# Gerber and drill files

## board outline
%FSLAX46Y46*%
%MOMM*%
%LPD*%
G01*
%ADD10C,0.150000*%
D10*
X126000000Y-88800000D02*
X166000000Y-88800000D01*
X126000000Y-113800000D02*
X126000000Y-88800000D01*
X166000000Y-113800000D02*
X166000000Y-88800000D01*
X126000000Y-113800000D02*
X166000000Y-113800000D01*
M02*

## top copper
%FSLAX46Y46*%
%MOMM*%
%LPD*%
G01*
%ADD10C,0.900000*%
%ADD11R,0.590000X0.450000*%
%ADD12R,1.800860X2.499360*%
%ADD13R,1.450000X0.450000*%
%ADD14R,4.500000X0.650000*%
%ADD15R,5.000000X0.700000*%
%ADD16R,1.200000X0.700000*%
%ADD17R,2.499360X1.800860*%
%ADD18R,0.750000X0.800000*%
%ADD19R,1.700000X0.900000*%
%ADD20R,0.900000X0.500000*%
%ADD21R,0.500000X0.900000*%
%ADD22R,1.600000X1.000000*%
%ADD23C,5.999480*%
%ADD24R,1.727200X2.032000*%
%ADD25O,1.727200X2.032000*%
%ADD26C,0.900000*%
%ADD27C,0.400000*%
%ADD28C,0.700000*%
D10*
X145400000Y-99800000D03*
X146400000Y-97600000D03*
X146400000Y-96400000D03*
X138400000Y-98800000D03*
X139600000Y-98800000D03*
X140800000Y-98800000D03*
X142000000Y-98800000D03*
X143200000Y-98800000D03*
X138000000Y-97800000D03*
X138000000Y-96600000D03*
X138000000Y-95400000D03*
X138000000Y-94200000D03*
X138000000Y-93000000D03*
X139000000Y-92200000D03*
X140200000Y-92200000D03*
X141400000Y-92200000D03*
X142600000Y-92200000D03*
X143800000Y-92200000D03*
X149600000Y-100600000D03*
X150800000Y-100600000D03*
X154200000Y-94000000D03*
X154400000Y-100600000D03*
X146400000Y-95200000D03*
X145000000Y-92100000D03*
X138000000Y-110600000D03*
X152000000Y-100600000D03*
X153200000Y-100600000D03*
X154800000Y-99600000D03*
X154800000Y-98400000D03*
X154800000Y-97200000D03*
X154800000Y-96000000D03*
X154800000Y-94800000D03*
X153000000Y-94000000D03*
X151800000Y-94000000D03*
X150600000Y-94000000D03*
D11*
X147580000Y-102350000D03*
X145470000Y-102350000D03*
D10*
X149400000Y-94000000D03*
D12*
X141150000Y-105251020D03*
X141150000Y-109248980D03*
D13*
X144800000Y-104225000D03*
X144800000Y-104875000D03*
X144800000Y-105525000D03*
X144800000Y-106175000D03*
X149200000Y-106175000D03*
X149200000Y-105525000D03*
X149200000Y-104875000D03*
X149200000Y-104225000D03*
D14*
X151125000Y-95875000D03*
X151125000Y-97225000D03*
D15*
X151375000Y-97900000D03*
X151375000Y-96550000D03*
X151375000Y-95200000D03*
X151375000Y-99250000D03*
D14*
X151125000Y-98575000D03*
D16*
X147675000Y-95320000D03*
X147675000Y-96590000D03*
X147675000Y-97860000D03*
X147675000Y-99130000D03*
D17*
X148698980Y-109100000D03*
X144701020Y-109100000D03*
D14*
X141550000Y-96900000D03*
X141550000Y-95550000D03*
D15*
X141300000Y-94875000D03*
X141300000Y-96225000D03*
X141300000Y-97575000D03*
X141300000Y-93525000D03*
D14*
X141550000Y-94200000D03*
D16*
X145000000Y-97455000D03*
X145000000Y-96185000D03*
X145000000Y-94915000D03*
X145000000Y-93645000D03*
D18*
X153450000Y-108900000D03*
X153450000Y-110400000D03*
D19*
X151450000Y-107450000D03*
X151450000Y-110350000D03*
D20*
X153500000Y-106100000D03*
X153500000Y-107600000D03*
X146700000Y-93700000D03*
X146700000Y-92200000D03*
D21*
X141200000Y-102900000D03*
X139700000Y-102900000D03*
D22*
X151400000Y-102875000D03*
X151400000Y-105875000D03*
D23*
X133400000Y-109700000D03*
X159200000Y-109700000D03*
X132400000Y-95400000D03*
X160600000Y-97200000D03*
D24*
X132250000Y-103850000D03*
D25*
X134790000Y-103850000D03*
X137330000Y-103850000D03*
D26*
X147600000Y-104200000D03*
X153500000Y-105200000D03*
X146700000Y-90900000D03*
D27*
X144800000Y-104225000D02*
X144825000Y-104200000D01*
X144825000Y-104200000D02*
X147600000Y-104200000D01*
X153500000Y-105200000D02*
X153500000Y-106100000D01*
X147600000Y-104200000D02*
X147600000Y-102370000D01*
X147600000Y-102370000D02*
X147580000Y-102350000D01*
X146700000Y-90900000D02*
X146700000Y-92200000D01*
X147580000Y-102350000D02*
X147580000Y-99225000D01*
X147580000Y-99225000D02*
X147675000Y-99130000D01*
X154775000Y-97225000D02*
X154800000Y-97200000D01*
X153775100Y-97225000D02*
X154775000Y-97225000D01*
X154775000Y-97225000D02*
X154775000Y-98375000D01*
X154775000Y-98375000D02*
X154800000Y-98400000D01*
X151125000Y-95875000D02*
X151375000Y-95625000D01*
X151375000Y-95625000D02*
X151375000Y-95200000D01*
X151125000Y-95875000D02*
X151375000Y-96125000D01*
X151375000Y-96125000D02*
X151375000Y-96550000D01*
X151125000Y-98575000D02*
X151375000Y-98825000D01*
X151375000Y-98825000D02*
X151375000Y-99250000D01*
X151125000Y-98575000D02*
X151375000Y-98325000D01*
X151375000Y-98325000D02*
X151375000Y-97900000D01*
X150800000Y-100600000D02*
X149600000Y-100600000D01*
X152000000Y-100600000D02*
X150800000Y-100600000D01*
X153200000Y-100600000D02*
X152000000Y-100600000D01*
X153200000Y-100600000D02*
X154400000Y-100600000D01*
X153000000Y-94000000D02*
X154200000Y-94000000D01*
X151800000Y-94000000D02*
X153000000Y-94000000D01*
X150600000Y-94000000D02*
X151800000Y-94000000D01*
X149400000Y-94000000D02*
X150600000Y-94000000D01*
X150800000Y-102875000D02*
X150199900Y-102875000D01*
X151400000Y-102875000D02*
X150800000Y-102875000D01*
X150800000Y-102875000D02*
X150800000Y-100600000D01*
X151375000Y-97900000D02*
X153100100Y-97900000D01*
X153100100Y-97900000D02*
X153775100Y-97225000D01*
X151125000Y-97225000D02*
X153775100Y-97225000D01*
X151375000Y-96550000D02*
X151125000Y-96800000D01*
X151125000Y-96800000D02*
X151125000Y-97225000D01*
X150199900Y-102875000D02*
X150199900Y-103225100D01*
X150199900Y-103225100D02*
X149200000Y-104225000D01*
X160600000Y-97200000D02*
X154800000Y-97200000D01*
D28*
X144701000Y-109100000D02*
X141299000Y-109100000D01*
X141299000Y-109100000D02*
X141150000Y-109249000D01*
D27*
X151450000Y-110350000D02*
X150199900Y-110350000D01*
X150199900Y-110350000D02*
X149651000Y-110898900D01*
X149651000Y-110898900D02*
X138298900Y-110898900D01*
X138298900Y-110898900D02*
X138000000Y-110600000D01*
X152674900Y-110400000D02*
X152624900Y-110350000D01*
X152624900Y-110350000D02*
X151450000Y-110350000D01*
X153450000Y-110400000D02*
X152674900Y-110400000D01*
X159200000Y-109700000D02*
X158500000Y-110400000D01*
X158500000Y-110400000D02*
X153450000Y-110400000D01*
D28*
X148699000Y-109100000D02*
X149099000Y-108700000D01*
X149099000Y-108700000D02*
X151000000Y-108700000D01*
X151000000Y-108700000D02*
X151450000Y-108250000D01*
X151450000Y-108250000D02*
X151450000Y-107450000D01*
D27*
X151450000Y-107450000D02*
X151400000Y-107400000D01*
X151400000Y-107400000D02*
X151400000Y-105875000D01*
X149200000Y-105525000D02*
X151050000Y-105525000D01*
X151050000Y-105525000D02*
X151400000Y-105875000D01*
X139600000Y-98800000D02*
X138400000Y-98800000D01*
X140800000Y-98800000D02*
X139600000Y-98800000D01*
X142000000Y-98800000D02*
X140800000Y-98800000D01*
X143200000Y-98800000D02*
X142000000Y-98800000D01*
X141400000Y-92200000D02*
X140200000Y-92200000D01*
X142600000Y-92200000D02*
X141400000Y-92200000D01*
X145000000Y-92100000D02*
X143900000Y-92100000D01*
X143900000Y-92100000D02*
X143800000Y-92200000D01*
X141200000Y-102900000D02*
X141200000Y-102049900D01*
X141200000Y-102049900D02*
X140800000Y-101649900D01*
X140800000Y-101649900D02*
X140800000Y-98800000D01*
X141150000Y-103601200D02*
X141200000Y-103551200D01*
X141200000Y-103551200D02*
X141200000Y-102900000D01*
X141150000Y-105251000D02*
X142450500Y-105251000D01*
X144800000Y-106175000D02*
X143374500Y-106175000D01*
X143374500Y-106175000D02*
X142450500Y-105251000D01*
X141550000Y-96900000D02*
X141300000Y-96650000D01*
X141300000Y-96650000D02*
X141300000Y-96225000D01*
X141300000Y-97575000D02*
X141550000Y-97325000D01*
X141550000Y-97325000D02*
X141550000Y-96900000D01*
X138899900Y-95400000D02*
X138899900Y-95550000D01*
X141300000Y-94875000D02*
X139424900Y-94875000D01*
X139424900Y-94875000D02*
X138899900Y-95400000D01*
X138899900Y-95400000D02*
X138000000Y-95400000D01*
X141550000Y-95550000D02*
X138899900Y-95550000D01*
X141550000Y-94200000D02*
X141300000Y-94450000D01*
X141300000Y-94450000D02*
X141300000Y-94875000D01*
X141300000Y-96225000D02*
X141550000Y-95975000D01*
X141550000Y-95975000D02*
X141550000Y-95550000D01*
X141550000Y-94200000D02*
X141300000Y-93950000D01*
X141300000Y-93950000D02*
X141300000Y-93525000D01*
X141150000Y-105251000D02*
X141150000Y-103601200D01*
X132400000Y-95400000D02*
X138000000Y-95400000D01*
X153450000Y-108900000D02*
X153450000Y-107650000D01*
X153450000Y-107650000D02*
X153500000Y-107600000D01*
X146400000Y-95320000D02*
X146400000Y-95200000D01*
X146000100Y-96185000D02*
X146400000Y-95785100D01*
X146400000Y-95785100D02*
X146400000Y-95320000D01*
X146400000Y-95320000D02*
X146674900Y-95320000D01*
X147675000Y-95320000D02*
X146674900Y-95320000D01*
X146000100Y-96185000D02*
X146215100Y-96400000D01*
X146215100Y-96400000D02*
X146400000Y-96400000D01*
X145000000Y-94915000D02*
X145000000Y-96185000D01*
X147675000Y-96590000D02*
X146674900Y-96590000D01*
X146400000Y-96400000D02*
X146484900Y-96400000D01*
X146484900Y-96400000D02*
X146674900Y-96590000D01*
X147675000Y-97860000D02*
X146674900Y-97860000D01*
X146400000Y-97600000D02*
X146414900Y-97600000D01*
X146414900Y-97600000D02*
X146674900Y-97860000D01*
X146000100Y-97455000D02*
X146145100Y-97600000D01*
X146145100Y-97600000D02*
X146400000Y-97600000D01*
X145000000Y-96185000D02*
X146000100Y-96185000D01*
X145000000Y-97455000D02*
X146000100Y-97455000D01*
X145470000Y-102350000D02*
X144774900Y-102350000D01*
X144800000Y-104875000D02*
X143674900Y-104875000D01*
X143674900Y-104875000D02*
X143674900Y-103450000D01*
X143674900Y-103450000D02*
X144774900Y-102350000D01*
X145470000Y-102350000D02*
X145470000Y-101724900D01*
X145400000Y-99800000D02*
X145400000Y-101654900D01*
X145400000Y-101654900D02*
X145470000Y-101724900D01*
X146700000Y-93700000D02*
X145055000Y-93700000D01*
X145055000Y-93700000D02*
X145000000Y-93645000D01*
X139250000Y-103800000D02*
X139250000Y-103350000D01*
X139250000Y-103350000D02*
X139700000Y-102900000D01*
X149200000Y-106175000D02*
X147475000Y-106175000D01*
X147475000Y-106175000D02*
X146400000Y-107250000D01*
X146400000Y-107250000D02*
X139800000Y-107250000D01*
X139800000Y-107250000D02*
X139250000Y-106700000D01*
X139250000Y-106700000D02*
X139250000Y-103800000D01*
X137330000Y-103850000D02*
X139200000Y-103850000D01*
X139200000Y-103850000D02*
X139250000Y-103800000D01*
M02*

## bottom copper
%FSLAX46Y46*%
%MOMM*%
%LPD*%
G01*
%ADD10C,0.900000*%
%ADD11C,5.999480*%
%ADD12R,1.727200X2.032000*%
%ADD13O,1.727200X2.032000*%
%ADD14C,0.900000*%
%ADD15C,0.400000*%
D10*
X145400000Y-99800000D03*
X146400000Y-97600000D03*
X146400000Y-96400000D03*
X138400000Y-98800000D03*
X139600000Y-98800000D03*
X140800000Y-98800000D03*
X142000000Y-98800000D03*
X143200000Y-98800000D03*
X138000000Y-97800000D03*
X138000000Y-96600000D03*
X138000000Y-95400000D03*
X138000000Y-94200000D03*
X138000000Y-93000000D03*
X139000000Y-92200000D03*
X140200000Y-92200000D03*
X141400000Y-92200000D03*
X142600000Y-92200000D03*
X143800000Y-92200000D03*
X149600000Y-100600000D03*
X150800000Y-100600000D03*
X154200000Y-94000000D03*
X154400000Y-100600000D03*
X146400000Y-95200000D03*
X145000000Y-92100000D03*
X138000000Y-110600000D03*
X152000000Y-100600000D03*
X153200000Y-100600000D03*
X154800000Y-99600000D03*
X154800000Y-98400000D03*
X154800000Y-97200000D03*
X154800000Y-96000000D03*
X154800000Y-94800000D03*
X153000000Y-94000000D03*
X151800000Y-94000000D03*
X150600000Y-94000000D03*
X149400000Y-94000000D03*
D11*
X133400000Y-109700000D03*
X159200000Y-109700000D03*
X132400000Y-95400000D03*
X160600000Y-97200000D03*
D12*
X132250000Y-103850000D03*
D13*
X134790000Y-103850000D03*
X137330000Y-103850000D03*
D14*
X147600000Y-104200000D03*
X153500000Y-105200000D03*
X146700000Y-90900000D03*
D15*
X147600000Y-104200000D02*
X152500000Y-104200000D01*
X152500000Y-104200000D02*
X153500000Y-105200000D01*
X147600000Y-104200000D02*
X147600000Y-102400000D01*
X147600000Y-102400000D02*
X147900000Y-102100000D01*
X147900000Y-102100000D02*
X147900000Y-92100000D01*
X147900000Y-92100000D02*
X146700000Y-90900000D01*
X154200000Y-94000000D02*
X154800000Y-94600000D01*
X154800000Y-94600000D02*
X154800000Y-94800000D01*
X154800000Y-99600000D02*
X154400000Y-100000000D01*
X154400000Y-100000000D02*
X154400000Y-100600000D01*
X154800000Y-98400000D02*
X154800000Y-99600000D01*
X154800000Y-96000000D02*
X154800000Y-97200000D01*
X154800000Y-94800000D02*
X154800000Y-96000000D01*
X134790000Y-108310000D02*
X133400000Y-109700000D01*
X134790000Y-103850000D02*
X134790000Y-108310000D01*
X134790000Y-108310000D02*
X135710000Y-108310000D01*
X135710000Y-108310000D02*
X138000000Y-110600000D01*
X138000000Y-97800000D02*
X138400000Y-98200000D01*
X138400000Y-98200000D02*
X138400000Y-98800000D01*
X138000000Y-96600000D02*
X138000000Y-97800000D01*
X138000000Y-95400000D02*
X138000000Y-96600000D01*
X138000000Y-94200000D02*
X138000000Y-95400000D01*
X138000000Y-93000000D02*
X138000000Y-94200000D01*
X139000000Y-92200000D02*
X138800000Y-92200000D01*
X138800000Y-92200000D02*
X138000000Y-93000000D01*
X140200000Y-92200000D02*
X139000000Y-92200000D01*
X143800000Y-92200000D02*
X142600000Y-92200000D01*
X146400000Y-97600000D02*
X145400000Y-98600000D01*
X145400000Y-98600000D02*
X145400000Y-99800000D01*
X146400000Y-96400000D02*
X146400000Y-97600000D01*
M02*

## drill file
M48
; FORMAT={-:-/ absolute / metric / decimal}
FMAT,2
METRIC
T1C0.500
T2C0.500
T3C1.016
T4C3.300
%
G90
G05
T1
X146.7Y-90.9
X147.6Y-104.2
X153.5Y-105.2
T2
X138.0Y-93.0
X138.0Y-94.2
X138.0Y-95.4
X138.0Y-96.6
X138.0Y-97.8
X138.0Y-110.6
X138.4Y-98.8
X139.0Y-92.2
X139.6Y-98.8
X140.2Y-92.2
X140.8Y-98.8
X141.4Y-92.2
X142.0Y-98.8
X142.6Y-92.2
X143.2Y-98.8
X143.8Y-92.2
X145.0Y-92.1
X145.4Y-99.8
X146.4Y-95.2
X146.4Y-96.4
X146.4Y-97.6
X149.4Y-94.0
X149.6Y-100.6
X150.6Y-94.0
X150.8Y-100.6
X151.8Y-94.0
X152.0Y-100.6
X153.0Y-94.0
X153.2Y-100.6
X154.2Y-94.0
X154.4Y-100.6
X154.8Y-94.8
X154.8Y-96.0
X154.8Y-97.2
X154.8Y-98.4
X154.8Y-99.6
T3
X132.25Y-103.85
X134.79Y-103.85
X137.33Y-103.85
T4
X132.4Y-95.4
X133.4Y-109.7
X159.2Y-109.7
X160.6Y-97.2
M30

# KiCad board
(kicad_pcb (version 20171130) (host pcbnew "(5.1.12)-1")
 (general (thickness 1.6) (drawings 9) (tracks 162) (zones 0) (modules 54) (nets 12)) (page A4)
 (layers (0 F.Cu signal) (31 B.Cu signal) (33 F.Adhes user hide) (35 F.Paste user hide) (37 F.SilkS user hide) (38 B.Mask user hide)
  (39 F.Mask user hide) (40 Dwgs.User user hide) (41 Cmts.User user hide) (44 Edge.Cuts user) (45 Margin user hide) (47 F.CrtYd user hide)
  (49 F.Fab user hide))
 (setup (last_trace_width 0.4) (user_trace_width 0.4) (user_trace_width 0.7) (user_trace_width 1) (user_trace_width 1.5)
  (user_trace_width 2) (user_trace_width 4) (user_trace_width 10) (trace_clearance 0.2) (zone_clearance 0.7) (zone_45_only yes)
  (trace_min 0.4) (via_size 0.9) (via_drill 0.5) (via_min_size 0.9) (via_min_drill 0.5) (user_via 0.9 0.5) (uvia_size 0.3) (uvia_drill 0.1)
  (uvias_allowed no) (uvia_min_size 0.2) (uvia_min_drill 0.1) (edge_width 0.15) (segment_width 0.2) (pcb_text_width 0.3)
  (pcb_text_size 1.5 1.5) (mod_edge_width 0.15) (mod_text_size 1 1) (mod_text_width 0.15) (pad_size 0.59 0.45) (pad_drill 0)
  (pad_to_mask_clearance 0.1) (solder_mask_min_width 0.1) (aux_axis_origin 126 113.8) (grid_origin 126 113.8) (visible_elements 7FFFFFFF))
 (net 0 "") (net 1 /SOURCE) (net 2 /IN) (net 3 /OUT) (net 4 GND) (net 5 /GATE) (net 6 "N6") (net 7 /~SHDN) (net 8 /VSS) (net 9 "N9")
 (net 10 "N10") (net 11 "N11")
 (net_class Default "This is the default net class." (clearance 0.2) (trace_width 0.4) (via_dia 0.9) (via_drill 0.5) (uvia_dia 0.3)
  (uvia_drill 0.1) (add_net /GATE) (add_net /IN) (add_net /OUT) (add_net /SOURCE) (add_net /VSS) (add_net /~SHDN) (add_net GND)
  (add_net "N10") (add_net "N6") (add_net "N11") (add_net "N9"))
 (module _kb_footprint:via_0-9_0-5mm (layer F.Cu) (at 145.4 99.8)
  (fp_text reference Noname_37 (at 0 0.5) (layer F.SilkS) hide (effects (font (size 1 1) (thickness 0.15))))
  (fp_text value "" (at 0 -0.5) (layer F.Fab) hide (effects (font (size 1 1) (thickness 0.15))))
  (pad 1 thru_hole circle (at 0 0) (size 0.9 0.9) (drill 0.5) (layers *.Cu) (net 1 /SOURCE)))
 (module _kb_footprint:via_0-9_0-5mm (layer F.Cu) (at 146.4 97.6)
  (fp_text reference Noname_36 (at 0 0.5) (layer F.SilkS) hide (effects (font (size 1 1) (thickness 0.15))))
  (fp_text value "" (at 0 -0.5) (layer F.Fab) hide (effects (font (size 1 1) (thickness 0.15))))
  (pad 1 thru_hole circle (at 0 0) (size 0.9 0.9) (drill 0.5) (layers *.Cu) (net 1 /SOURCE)))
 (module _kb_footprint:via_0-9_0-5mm (layer F.Cu) (at 146.4 96.4)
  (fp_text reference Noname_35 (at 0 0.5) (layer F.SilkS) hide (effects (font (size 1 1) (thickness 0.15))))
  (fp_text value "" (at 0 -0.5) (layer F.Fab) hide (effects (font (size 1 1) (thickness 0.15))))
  (pad 1 thru_hole circle (at 0 0) (size 0.9 0.9) (drill 0.5) (layers *.Cu) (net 1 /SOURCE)))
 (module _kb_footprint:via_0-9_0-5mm (layer F.Cu) (at 138.4 98.8)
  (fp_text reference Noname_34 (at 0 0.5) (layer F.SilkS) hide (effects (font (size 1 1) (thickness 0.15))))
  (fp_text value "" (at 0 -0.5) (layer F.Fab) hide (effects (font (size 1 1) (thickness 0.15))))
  (pad 1 thru_hole circle (at 0 0) (size 0.9 0.9) (drill 0.5) (layers *.Cu) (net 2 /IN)))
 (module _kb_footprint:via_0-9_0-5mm (layer F.Cu) (at 139.6 98.8)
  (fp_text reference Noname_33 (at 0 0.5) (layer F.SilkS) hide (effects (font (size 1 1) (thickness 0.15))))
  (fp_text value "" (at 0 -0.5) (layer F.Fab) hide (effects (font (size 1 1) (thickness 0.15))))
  (pad 1 thru_hole circle (at 0 0) (size 0.9 0.9) (drill 0.5) (layers *.Cu) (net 2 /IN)))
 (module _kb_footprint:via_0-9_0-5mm (layer F.Cu) (at 140.8 98.8)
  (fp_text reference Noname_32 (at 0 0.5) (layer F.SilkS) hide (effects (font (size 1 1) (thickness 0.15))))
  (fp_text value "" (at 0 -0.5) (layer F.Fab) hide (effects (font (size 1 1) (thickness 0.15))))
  (pad 1 thru_hole circle (at 0 0) (size 0.9 0.9) (drill 0.5) (layers *.Cu) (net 2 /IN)))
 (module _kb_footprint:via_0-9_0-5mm (layer F.Cu) (at 142 98.8)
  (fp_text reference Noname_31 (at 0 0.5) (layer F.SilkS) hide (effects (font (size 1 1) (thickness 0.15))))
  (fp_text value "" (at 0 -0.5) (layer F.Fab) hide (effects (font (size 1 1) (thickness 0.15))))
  (pad 1 thru_hole circle (at 0 0) (size 0.9 0.9) (drill 0.5) (layers *.Cu) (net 2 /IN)))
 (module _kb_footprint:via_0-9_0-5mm (layer F.Cu) (at 143.2 98.8)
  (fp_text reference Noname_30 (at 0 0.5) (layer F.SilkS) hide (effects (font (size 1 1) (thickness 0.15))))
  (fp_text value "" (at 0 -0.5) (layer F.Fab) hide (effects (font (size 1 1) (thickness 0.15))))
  (pad 1 thru_hole circle (at 0 0) (size 0.9 0.9) (drill 0.5) (layers *.Cu) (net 2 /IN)))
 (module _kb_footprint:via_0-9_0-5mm (layer F.Cu) (at 138 97.8)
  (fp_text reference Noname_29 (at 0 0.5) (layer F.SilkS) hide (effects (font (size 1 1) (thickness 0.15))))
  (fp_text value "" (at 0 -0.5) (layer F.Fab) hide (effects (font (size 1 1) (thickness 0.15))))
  (pad 1 thru_hole circle (at 0 0) (size 0.9 0.9) (drill 0.5) (layers *.Cu) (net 2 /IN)))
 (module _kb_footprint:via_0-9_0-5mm (layer F.Cu) (at 138 96.6)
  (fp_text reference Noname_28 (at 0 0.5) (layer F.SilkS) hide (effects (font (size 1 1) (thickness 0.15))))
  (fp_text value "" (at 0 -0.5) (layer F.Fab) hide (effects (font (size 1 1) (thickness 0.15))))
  (pad 1 thru_hole circle (at 0 0) (size 0.9 0.9) (drill 0.5) (layers *.Cu) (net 2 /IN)))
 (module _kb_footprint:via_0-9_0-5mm (layer F.Cu) (at 138 95.4)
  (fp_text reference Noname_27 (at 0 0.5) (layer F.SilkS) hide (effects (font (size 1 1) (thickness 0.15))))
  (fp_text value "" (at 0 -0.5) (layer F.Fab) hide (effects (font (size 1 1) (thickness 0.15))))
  (pad 1 thru_hole circle (at 0 0) (size 0.9 0.9) (drill 0.5) (layers *.Cu) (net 2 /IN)))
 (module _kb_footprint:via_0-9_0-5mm (layer F.Cu) (at 138 94.2)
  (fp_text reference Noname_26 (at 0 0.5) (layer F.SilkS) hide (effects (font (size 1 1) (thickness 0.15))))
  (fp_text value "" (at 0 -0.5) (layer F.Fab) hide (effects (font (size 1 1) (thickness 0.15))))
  (pad 1 thru_hole circle (at 0 0) (size 0.9 0.9) (drill 0.5) (layers *.Cu) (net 2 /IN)))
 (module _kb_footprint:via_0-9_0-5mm (layer F.Cu) (at 138 93)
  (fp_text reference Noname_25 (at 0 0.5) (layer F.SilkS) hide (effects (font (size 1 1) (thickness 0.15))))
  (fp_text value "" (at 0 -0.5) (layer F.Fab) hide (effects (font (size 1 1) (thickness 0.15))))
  (pad 1 thru_hole circle (at 0 0) (size 0.9 0.9) (drill 0.5) (layers *.Cu) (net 2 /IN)))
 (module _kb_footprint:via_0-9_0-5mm (layer F.Cu) (at 139 92.2)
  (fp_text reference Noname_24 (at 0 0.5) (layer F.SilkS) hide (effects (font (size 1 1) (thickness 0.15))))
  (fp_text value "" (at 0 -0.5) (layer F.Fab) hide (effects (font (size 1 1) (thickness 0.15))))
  (pad 1 thru_hole circle (at 0 0) (size 0.9 0.9) (drill 0.5) (layers *.Cu) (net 2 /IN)))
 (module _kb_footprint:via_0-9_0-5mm (layer F.Cu) (at 140.2 92.2)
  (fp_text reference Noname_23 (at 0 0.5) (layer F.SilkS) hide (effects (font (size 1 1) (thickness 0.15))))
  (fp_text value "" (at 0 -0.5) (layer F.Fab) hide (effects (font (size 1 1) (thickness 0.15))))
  (pad 1 thru_hole circle (at 0 0) (size 0.9 0.9) (drill 0.5) (layers *.Cu) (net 2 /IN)))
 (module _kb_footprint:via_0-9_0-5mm (layer F.Cu) (at 141.4 92.2)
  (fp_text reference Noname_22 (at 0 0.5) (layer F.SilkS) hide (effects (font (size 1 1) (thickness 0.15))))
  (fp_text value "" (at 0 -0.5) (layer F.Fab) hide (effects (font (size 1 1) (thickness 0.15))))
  (pad 1 thru_hole circle (at 0 0) (size 0.9 0.9) (drill 0.5) (layers *.Cu) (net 2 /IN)))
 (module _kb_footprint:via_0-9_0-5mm (layer F.Cu) (at 142.6 92.2)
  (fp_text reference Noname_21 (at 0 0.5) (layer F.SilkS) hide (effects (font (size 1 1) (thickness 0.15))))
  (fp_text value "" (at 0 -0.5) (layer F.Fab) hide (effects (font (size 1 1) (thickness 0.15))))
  (pad 1 thru_hole circle (at 0 0) (size 0.9 0.9) (drill 0.5) (layers *.Cu) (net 2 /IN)))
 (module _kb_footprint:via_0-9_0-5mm (layer F.Cu) (at 143.8 92.2)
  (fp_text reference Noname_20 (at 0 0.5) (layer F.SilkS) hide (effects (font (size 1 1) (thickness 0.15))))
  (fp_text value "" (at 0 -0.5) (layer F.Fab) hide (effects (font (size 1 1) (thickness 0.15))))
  (pad 1 thru_hole circle (at 0 0) (size 0.9 0.9) (drill 0.5) (layers *.Cu) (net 2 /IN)))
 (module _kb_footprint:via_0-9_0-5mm (layer F.Cu) (at 149.6 100.6)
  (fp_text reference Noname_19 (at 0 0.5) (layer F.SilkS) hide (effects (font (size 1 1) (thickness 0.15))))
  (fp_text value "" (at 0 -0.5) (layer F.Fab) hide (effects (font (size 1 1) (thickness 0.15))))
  (pad 1 thru_hole circle (at 0 0) (size 0.9 0.9) (drill 0.5) (layers *.Cu) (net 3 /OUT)))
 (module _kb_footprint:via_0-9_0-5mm (layer F.Cu) (at 150.8 100.6)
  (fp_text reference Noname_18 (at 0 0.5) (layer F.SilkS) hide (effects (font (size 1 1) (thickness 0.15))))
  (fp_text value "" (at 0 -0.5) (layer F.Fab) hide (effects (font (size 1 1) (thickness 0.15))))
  (pad 1 thru_hole circle (at 0 0) (size 0.9 0.9) (drill 0.5) (layers *.Cu) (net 3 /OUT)))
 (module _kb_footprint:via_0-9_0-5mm (layer F.Cu) (at 154.2 94)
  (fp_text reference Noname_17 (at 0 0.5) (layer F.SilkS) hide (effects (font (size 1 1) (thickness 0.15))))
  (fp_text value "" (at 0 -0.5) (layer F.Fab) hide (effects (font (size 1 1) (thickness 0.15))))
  (pad 1 thru_hole circle (at 0 0) (size 0.9 0.9) (drill 0.5) (layers *.Cu) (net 3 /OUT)))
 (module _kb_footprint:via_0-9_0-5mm (layer F.Cu) (at 154.4 100.6)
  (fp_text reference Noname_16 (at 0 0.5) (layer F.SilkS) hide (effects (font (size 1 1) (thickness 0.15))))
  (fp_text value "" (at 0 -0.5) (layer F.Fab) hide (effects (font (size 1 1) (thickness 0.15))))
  (pad 1 thru_hole circle (at 0 0) (size 0.9 0.9) (drill 0.5) (layers *.Cu) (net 3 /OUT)))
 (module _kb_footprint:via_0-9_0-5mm (layer F.Cu) (at 146.4 95.2)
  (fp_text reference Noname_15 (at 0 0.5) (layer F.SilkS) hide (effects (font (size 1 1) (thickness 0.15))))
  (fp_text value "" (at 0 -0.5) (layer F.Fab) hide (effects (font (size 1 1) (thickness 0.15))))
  (pad 1 thru_hole circle (at 0 0) (size 0.9 0.9) (drill 0.5) (layers *.Cu) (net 1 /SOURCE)))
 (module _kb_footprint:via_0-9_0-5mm (layer F.Cu) (at 145 92.1)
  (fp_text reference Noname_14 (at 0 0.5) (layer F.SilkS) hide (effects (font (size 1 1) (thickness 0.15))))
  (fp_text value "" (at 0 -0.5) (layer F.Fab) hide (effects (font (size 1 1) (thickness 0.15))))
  (pad 1 thru_hole circle (at 0 0) (size 0.9 0.9) (drill 0.5) (layers *.Cu) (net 2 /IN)))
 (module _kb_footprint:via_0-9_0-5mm (layer F.Cu) (at 138 110.6)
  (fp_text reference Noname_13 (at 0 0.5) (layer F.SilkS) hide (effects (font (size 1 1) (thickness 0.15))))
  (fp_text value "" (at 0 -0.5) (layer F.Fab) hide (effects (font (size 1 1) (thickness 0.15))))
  (pad 1 thru_hole circle (at 0 0) (size 0.9 0.9) (drill 0.5) (layers *.Cu) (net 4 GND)))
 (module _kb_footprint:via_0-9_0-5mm (layer F.Cu) (at 152 100.6)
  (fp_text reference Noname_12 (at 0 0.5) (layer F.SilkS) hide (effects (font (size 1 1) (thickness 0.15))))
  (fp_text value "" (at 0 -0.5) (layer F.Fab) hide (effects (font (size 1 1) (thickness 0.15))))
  (pad 1 thru_hole circle (at 0 0) (size 0.9 0.9) (drill 0.5) (layers *.Cu) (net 3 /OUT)))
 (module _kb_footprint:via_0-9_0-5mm (layer F.Cu) (at 153.2 100.6)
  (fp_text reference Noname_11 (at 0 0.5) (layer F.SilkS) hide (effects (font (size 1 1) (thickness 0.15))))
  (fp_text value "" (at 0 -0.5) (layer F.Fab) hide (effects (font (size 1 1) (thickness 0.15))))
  (pad 1 thru_hole circle (at 0 0) (size 0.9 0.9) (drill 0.5) (layers *.Cu) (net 3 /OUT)))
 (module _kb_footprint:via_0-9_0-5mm (layer F.Cu) (at 154.8 99.6)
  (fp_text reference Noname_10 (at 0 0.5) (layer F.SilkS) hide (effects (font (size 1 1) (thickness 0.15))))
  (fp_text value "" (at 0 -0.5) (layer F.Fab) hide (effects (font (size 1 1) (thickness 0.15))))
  (pad 1 thru_hole circle (at 0 0) (size 0.9 0.9) (drill 0.5) (layers *.Cu) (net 3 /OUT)))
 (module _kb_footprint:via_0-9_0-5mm (layer F.Cu) (at 154.8 98.4)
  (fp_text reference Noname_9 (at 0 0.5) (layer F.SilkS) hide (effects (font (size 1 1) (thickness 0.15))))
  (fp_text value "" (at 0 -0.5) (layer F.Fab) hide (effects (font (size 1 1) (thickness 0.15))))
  (pad 1 thru_hole circle (at 0 0) (size 0.9 0.9) (drill 0.5) (layers *.Cu) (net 3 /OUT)))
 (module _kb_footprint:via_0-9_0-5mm (layer F.Cu) (at 154.8 97.2)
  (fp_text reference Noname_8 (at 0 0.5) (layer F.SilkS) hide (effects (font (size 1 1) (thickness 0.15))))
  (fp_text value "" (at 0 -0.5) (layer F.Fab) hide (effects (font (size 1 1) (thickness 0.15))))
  (pad 1 thru_hole circle (at 0 0) (size 0.9 0.9) (drill 0.5) (layers *.Cu) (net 3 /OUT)))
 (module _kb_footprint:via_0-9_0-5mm (layer F.Cu) (at 154.8 96)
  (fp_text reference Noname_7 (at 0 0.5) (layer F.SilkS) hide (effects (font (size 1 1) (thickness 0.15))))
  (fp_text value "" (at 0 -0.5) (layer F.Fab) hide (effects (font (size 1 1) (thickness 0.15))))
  (pad 1 thru_hole circle (at 0 0) (size 0.9 0.9) (drill 0.5) (layers *.Cu) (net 3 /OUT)))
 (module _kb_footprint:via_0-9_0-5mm (layer F.Cu) (at 154.8 94.8)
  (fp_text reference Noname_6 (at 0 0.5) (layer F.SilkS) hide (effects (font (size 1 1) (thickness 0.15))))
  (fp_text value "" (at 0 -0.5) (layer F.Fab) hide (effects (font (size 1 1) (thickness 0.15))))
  (pad 1 thru_hole circle (at 0 0) (size 0.9 0.9) (drill 0.5) (layers *.Cu) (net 3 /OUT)))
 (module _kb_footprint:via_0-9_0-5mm (layer F.Cu) (at 153 94)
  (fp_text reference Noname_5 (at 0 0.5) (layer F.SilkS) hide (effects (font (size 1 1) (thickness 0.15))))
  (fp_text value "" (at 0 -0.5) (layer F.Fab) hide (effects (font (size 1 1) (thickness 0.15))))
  (pad 1 thru_hole circle (at 0 0) (size 0.9 0.9) (drill 0.5) (layers *.Cu) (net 3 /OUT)))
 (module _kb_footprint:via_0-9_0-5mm (layer F.Cu) (at 151.8 94)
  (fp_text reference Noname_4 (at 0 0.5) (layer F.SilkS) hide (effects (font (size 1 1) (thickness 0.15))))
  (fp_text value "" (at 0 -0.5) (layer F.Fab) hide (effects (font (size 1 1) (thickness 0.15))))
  (pad 1 thru_hole circle (at 0 0) (size 0.9 0.9) (drill 0.5) (layers *.Cu) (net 3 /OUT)))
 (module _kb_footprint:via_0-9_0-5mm (layer F.Cu) (at 150.6 94)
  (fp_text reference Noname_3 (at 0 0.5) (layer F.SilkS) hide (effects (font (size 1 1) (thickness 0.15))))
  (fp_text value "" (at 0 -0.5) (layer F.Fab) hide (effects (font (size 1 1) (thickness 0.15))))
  (pad 1 thru_hole circle (at 0 0) (size 0.9 0.9) (drill 0.5) (layers *.Cu) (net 3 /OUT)))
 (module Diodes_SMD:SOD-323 (layer F.Cu) (at 146.525 102.35 180)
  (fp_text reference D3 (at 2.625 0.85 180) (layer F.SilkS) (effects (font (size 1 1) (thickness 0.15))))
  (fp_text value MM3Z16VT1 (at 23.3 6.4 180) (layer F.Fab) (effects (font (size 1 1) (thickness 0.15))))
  (pad 1 smd rect (at -1.055 0 180) (size 0.59 0.45) (layers F.Cu F.Paste F.Mask) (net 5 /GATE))
  (pad 2 smd rect (at 1.055 0 180) (size 0.59 0.45) (layers F.Cu F.Paste F.Mask) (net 1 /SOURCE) (zone_connect 1)))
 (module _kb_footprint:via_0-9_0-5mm (layer F.Cu) (at 149.4 94)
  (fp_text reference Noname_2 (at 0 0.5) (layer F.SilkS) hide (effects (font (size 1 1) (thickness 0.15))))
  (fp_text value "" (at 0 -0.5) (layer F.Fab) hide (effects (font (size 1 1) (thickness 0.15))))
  (pad 1 thru_hole circle (at 0 0) (size 0.9 0.9) (drill 0.5) (layers *.Cu) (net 3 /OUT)))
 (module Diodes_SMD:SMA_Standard (layer F.Cu) (at 141.15 107.25 270)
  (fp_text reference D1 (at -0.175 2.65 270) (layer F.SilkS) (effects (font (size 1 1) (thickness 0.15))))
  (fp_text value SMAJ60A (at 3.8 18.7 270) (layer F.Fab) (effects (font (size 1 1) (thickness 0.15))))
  (pad 1 smd rect (at -1.99898 0 270) (size 2.49936 1.80086) (layers F.Cu F.Paste F.Mask) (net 2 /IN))
  (pad 2 smd rect (at 1.99898 0 270) (size 2.49936 1.80086) (layers F.Cu F.Paste F.Mask) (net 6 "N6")))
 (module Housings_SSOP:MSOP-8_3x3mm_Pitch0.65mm (layer F.Cu) (at 147 105.2)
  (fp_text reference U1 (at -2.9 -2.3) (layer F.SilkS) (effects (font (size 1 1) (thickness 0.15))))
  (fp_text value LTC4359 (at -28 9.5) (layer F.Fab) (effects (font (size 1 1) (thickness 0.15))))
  (pad 1 smd rect (at -2.2 -0.975) (size 1.45 0.45) (layers F.Cu F.Paste F.Mask) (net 5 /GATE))
  (pad 2 smd rect (at -2.2 -0.325) (size 1.45 0.45) (layers F.Cu F.Paste F.Mask) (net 1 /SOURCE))
  (pad 3 smd rect (at -2.2 0.325) (size 1.45 0.45) (layers F.Cu F.Paste F.Mask))
  (pad 4 smd rect (at -2.2 0.975) (size 1.45 0.45) (layers F.Cu F.Paste F.Mask) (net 2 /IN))
  (pad 5 smd rect (at 2.2 0.975) (size 1.45 0.45) (layers F.Cu F.Paste F.Mask) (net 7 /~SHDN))
  (pad 6 smd rect (at 2.2 0.325) (size 1.45 0.45) (layers F.Cu F.Paste F.Mask) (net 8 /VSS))
  (pad 7 smd rect (at 2.2 -0.325) (size 1.45 0.45) (layers F.Cu F.Paste F.Mask))
  (pad 8 smd rect (at 2.2 -0.975) (size 1.45 0.45) (layers F.Cu F.Paste F.Mask) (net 3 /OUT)))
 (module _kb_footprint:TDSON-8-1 (layer F.Cu) (at 150.475 97.225)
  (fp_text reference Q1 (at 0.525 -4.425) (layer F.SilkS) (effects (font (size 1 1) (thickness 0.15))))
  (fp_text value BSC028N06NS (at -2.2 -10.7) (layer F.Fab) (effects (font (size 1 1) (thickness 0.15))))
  (pad 7 smd rect (at 0.65 -1.35) (size 4.5 0.65) (layers F.Cu F.Paste F.Mask) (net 3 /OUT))
  (pad 6 smd rect (at 0.65 0) (size 4.5 0.65) (layers F.Cu F.Paste F.Mask) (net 3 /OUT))
  (pad 6 smd rect (at 0.9 0.675) (size 5 0.7) (layers F.Cu F.Paste F.Mask) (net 3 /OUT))
  (pad 7 smd rect (at 0.9 -0.675) (size 5 0.7) (layers F.Cu F.Paste F.Mask) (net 3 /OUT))
  (pad 8 smd rect (at 0.9 -2.025) (size 5 0.7) (layers F.Cu F.Paste F.Mask) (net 3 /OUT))
  (pad 5 smd rect (at 0.9 2.025) (size 5 0.7) (layers F.Cu F.Paste F.Mask) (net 3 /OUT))
  (pad 5 smd rect (at 0.65 1.35) (size 4.5 0.65) (layers F.Cu F.Paste F.Mask) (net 3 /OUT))
  (pad 1 smd rect (at -2.8 -1.905) (size 1.2 0.7) (layers F.Cu F.Paste F.Mask) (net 1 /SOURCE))
  (pad 2 smd rect (at -2.8 -0.635) (size 1.2 0.7) (layers F.Cu F.Paste F.Mask) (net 1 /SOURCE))
  (pad 3 smd rect (at -2.8 0.635) (size 1.2 0.7) (layers F.Cu F.Paste F.Mask) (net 1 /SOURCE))
  (pad 4 smd rect (at -2.8 1.905) (size 1.2 0.7) (layers F.Cu F.Paste F.Mask) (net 5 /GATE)))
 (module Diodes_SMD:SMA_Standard (layer F.Cu) (at 146.7 109.1 180)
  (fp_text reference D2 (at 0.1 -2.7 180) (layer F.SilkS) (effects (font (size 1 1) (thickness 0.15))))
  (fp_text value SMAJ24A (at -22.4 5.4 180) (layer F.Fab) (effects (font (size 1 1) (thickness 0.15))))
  (pad 1 smd rect (at -1.99898 0 180) (size 2.49936 1.80086) (layers F.Cu F.Paste F.Mask) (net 8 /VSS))
  (pad 2 smd rect (at 1.99898 0 180) (size 2.49936 1.80086) (layers F.Cu F.Paste F.Mask) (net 6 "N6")))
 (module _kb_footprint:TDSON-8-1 (layer F.Cu) (at 142.2 95.55 180)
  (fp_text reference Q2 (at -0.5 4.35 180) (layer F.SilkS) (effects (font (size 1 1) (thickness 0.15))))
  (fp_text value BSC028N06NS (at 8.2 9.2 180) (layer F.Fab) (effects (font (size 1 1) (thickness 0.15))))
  (pad 7 smd rect (at 0.65 -1.35 180) (size 4.5 0.65) (layers F.Cu F.Paste F.Mask) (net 2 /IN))
  (pad 6 smd rect (at 0.65 0 180) (size 4.5 0.65) (layers F.Cu F.Paste F.Mask) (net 2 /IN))
  (pad 6 smd rect (at 0.9 0.675 180) (size 5 0.7) (layers F.Cu F.Paste F.Mask) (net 2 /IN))
  (pad 7 smd rect (at 0.9 -0.675 180) (size 5 0.7) (layers F.Cu F.Paste F.Mask) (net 2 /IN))
  (pad 8 smd rect (at 0.9 -2.025 180) (size 5 0.7) (layers F.Cu F.Paste F.Mask) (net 2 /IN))
  (pad 5 smd rect (at 0.9 2.025 180) (size 5 0.7) (layers F.Cu F.Paste F.Mask) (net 2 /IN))
  (pad 5 smd rect (at 0.65 1.35 180) (size 4.5 0.65) (layers F.Cu F.Paste F.Mask) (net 2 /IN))
  (pad 1 smd rect (at -2.8 -1.905 180) (size 1.2 0.7) (layers F.Cu F.Paste F.Mask) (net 1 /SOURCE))
  (pad 2 smd rect (at -2.8 -0.635 180) (size 1.2 0.7) (layers F.Cu F.Paste F.Mask) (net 1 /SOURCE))
  (pad 3 smd rect (at -2.8 0.635 180) (size 1.2 0.7) (layers F.Cu F.Paste F.Mask) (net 1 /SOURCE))
  (pad 4 smd rect (at -2.8 1.905 180) (size 1.2 0.7) (layers F.Cu F.Paste F.Mask) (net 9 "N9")))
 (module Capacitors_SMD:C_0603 (layer F.Cu) (at 153.45 109.65 270)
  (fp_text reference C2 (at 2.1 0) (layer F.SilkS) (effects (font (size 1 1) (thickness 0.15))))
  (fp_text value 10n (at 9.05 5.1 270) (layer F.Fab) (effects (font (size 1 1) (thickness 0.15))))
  (pad 1 smd rect (at -0.75 0 270) (size 0.8 0.75) (layers F.Cu F.Paste F.Mask) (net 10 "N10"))
  (pad 2 smd rect (at 0.75 0 270) (size 0.8 0.75) (layers F.Cu F.Paste F.Mask) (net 4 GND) (zone_connect 1)))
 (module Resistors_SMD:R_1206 (layer F.Cu) (at 151.45 108.9 270)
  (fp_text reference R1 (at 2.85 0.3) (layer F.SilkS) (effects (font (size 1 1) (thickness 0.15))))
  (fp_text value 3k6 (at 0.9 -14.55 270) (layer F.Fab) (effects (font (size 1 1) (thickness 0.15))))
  (pad 1 smd rect (at -1.45 0 270) (size 0.9 1.7) (layers F.Cu F.Paste F.Mask) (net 8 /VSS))
  (pad 2 smd rect (at 1.45 0 270) (size 0.9 1.7) (layers F.Cu F.Paste F.Mask) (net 4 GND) (zone_connect 1)))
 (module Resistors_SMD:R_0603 (layer F.Cu) (at 153.5 106.85 270)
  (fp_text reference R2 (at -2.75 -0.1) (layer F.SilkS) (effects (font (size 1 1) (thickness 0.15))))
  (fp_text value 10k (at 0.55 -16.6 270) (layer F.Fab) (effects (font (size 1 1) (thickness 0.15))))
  (pad 1 smd rect (at -0.75 0 270) (size 0.5 0.9) (layers F.Cu F.Paste F.Mask) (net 5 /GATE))
  (pad 2 smd rect (at 0.75 0 270) (size 0.5 0.9) (layers F.Cu F.Paste F.Mask) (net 10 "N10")))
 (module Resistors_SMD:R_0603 (layer F.Cu) (at 146.7 92.95 90)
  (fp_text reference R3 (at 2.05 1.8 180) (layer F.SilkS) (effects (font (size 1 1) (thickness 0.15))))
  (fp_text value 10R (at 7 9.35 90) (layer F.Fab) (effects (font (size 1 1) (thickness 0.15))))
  (pad 1 smd rect (at -0.75 0 90) (size 0.5 0.9) (layers F.Cu F.Paste F.Mask) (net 9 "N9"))
  (pad 2 smd rect (at 0.75 0 90) (size 0.5 0.9) (layers F.Cu F.Paste F.Mask) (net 5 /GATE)))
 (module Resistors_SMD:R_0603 (layer F.Cu) (at 140.45 102.9 180)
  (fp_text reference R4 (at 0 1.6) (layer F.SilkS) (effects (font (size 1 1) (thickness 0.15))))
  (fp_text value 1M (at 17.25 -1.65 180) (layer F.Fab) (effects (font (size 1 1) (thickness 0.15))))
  (pad 1 smd rect (at -0.75 0 180) (size 0.5 0.9) (layers F.Cu F.Paste F.Mask) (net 2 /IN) (zone_connect 1))
  (pad 2 smd rect (at 0.75 0 180) (size 0.5 0.9) (layers F.Cu F.Paste F.Mask) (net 7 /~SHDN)))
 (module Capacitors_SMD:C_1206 (layer F.Cu) (at 151.4 104.375 270)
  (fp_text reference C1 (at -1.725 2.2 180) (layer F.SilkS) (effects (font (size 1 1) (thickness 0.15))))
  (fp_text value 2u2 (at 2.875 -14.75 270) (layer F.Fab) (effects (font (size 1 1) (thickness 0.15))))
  (pad 1 smd rect (at -1.5 0 270) (size 1 1.6) (layers F.Cu F.Paste F.Mask) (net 3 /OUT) (zone_connect 1))
  (pad 2 smd rect (at 1.5 0 270) (size 1 1.6) (layers F.Cu F.Paste F.Mask) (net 8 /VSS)))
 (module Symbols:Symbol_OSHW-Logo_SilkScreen (layer F.Cu) (at 174 87)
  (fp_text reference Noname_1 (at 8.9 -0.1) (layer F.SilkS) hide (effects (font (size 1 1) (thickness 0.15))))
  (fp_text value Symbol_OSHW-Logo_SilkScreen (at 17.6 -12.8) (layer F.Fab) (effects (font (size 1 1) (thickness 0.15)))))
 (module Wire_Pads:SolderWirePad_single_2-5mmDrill (layer F.Cu) (at 133.4 109.7)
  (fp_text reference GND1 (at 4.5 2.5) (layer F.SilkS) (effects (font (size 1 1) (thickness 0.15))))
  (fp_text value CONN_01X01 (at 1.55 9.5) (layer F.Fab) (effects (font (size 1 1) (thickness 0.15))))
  (pad 1 thru_hole circle (at 0 0) (size 5.99948 5.99948) (drill 3.3) (layers *.Cu *.Mask F.SilkS) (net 4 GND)))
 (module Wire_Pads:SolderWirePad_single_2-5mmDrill (layer F.Cu) (at 159.2 109.7)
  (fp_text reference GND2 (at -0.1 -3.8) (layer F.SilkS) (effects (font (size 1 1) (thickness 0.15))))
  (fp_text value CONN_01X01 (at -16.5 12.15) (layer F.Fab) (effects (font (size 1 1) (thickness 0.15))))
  (pad 1 thru_hole circle (at 0 0) (size 5.99948 5.99948) (drill 3.3) (layers *.Cu *.Mask F.SilkS) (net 4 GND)))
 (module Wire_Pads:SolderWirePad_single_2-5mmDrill (layer F.Cu) (at 132.4 95.4)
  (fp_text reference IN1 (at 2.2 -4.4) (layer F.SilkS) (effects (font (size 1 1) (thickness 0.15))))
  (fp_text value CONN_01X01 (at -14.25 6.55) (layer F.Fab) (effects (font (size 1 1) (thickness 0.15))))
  (pad 1 thru_hole circle (at 0 0) (size 5.99948 5.99948) (drill 3.3) (layers *.Cu *.Mask F.SilkS) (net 2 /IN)))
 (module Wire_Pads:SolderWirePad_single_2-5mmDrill (layer F.Cu) (at 160.6 97.2)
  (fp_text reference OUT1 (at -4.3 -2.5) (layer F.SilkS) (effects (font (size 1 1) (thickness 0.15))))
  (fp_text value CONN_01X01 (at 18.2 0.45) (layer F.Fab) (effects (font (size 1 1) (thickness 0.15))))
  (pad 1 thru_hole circle (at 0 0) (size 5.99948 5.99948) (drill 3.3) (layers *.Cu *.Mask F.SilkS) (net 3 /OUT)))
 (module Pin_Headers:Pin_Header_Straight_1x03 (layer F.Cu) (at 132.25 103.85 90)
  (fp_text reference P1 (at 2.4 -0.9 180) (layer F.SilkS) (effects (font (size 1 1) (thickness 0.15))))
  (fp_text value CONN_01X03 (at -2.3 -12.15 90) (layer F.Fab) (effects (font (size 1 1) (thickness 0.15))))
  (pad 1 thru_hole rect (at 0 0 90) (size 2.032 1.7272) (drill 1.016) (layers *.Cu *.Mask F.SilkS) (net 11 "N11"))
  (pad 2 thru_hole oval (at 0 2.54 90) (size 2.032 1.7272) (drill 1.016) (layers *.Cu *.Mask F.SilkS) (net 4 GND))
  (pad 3 thru_hole oval (at 0 5.08 90) (size 2.032 1.7272) (drill 1.016) (layers *.Cu *.Mask F.SilkS) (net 7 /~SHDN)))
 (gr_line (start 126 88.8) (end 166 88.8) (angle 90) (layer Edge.Cuts) (width 0.15))
 (gr_line (start 126 113.8) (end 126 88.8) (angle 90) (layer Edge.Cuts) (width 0.15))
 (gr_line (start 166 113.8) (end 166 88.8) (angle 90) (layer Edge.Cuts) (width 0.15))
 (gr_line (start 126 113.8) (end 166 113.8) (angle 90) (layer Edge.Cuts) (width 0.15))
 (segment (start 144.8 104.225) (end 144.825 104.2) (width 0.4) (layer F.Cu) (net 5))
 (segment (start 144.825 104.2) (end 147.6 104.2) (width 0.4) (layer F.Cu) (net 5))
 (segment (start 147.6 104.2) (end 152.5 104.2) (width 0.4) (layer B.Cu) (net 5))
 (segment (start 152.5 104.2) (end 153.5 105.2) (width 0.4) (layer B.Cu) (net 5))
 (segment (start 153.5 105.2) (end 153.5 106.1) (width 0.4) (layer F.Cu) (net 5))
 (segment (start 147.6 104.2) (end 147.6 102.37) (width 0.4) (layer F.Cu) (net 5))
 (segment (start 147.6 102.37) (end 147.58 102.35) (width 0.4) (layer F.Cu) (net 5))
 (segment (start 146.7 90.9) (end 146.7 92.2) (width 0.4) (layer F.Cu) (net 5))
 (segment (start 147.6 104.2) (end 147.6 102.4) (width 0.4) (layer B.Cu) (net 5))
 (segment (start 147.6 102.4) (end 147.9 102.1) (width 0.4) (layer B.Cu) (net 5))
 (segment (start 147.9 102.1) (end 147.9 92.1) (width 0.4) (layer B.Cu) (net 5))
 (segment (start 147.9 92.1) (end 146.7 90.9) (width 0.4) (layer B.Cu) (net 5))
 (segment (start 147.58 102.35) (end 147.58 99.225) (width 0.4) (layer F.Cu) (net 5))
 (segment (start 147.58 99.225) (end 147.675 99.13) (width 0.4) (layer F.Cu) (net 5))
 (via (at 147.6 104.2) (size 0.9) (layers F.Cu B.Cu) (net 5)) (via (at 153.5 105.2) (size 0.9) (layers F.Cu B.Cu) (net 5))
 (via (at 146.7 90.9) (size 0.9) (layers F.Cu B.Cu) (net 5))
 (segment (start 154.775 97.225) (end 154.8 97.2) (width 0.4) (layer F.Cu) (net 3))
 (segment (start 153.7751 97.225) (end 154.775 97.225) (width 0.4) (layer F.Cu) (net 3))
 (segment (start 154.775 97.225) (end 154.775 98.375) (width 0.4) (layer F.Cu) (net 3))
 (segment (start 154.775 98.375) (end 154.8 98.4) (width 0.4) (layer F.Cu) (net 3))
 (segment (start 151.125 95.875) (end 151.375 95.625) (width 0.4) (layer F.Cu) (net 3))
 (segment (start 151.375 95.625) (end 151.375 95.2) (width 0.4) (layer F.Cu) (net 3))
 (segment (start 151.125 95.875) (end 151.375 96.125) (width 0.4) (layer F.Cu) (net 3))
 (segment (start 151.375 96.125) (end 151.375 96.55) (width 0.4) (layer F.Cu) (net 3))
 (segment (start 151.125 98.575) (end 151.375 98.825) (width 0.4) (layer F.Cu) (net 3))
 (segment (start 151.375 98.825) (end 151.375 99.25) (width 0.4) (layer F.Cu) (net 3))
 (segment (start 151.125 98.575) (end 151.375 98.325) (width 0.4) (layer F.Cu) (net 3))
 (segment (start 151.375 98.325) (end 151.375 97.9) (width 0.4) (layer F.Cu) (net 3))
 (segment (start 150.8 100.6) (end 149.6 100.6) (width 0.4) (layer F.Cu) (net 3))
 (segment (start 152 100.6) (end 150.8 100.6) (width 0.4) (layer F.Cu) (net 3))
 (segment (start 154.2 94) (end 154.8 94.6) (width 0.4) (layer B.Cu) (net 3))
 (segment (start 154.8 94.6) (end 154.8 94.8) (width 0.4) (layer B.Cu) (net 3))
 (segment (start 153.2 100.6) (end 152 100.6) (width 0.4) (layer F.Cu) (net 3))
 (segment (start 153.2 100.6) (end 154.4 100.6) (width 0.4) (layer F.Cu) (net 3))
 (segment (start 154.8 99.6) (end 154.4 100) (width 0.4) (layer B.Cu) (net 3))
 (segment (start 154.4 100) (end 154.4 100.6) (width 0.4) (layer B.Cu) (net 3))
 (segment (start 154.8 98.4) (end 154.8 99.6) (width 0.4) (layer B.Cu) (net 3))
 (segment (start 154.8 96) (end 154.8 97.2) (width 0.4) (layer B.Cu) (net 3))
 (segment (start 154.8 94.8) (end 154.8 96) (width 0.4) (layer B.Cu) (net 3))
 (segment (start 153 94) (end 154.2 94) (width 0.4) (layer F.Cu) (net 3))
 (segment (start 151.8 94) (end 153 94) (width 0.4) (layer F.Cu) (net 3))
 (segment (start 150.6 94) (end 151.8 94) (width 0.4) (layer F.Cu) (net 3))
 (segment (start 149.4 94) (end 150.6 94) (width 0.4) (layer F.Cu) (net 3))
 (segment (start 150.8 102.875) (end 150.1999 102.875) (width 0.4) (layer F.Cu) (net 3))
 (segment (start 151.4 102.875) (end 150.8 102.875) (width 0.4) (layer F.Cu) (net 3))
 (segment (start 150.8 102.875) (end 150.8 100.6) (width 0.4) (layer F.Cu) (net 3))
 (segment (start 151.375 97.9) (end 153.1001 97.9) (width 0.4) (layer F.Cu) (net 3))
 (segment (start 153.1001 97.9) (end 153.7751 97.225) (width 0.4) (layer F.Cu) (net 3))
 (segment (start 151.125 97.225) (end 153.7751 97.225) (width 0.4) (layer F.Cu) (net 3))
 (segment (start 151.375 96.55) (end 151.125 96.8) (width 0.4) (layer F.Cu) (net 3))
 (segment (start 151.125 96.8) (end 151.125 97.225) (width 0.4) (layer F.Cu) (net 3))
 (segment (start 150.1999 102.875) (end 150.1999 103.2251) (width 0.4) (layer F.Cu) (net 3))
 (segment (start 150.1999 103.2251) (end 149.2 104.225) (width 0.4) (layer F.Cu) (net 3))
 (segment (start 160.6 97.2) (end 154.8 97.2) (width 0.4) (layer F.Cu) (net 3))
 (segment (start 144.701 109.1) (end 141.299 109.1) (width 0.7) (layer F.Cu) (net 6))
 (segment (start 141.299 109.1) (end 141.15 109.249) (width 0.7) (layer F.Cu) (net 6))
 (segment (start 134.79 108.31) (end 133.4 109.7) (width 0.4) (layer B.Cu) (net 4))
 (segment (start 134.79 103.85) (end 134.79 108.31) (width 0.4) (layer B.Cu) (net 4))
 (segment (start 134.79 108.31) (end 135.71 108.31) (width 0.4) (layer B.Cu) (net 4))
 (segment (start 135.71 108.31) (end 138 110.6) (width 0.4) (layer B.Cu) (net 4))
 (segment (start 151.45 110.35) (end 150.1999 110.35) (width 0.4) (layer F.Cu) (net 4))
 (segment (start 150.1999 110.35) (end 149.651 110.8989) (width 0.4) (layer F.Cu) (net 4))
 (segment (start 149.651 110.8989) (end 138.2989 110.8989) (width 0.4) (layer F.Cu) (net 4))
 (segment (start 138.2989 110.8989) (end 138 110.6) (width 0.4) (layer F.Cu) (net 4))
 (segment (start 152.6749 110.4) (end 152.6249 110.35) (width 0.4) (layer F.Cu) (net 4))
 (segment (start 152.6249 110.35) (end 151.45 110.35) (width 0.4) (layer F.Cu) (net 4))
 (segment (start 153.45 110.4) (end 152.6749 110.4) (width 0.4) (layer F.Cu) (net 4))
 (segment (start 159.2 109.7) (end 158.5 110.4) (width 0.4) (layer F.Cu) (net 4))
 (segment (start 158.5 110.4) (end 153.45 110.4) (width 0.4) (layer F.Cu) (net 4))
 (segment (start 148.699 109.1) (end 149.099 108.7) (width 0.7) (layer F.Cu) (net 8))
 (segment (start 149.099 108.7) (end 151 108.7) (width 0.7) (layer F.Cu) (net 8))
 (segment (start 151 108.7) (end 151.45 108.25) (width 0.7) (layer F.Cu) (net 8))
 (segment (start 151.45 108.25) (end 151.45 107.45) (width 0.7) (layer F.Cu) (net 8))
 (segment (start 151.45 107.45) (end 151.4 107.4) (width 0.4) (layer F.Cu) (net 8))
 (segment (start 151.4 107.4) (end 151.4 105.875) (width 0.4) (layer F.Cu) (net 8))
 (segment (start 149.2 105.525) (end 151.05 105.525) (width 0.4) (layer F.Cu) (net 8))
 (segment (start 151.05 105.525) (end 151.4 105.875) (width 0.4) (layer F.Cu) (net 8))
 (segment (start 139.6 98.8) (end 138.4 98.8) (width 0.4) (layer F.Cu) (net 2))
 (segment (start 140.8 98.8) (end 139.6 98.8) (width 0.4) (layer F.Cu) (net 2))
 (segment (start 142 98.8) (end 140.8 98.8) (width 0.4) (layer F.Cu) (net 2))
 (segment (start 143.2 98.8) (end 142 98.8) (width 0.4) (layer F.Cu) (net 2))
 (segment (start 138 97.8) (end 138.4 98.2) (width 0.4) (layer B.Cu) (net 2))
 (segment (start 138.4 98.2) (end 138.4 98.8) (width 0.4) (layer B.Cu) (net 2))
 (segment (start 138 96.6) (end 138 97.8) (width 0.4) (layer B.Cu) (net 2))
 (segment (start 138 95.4) (end 138 96.6) (width 0.4) (layer B.Cu) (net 2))
 (segment (start 138 94.2) (end 138 95.4) (width 0.4) (layer B.Cu) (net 2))
 (segment (start 138 93) (end 138 94.2) (width 0.4) (layer B.Cu) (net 2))
 (segment (start 139 92.2) (end 138.8 92.2) (width 0.4) (layer B.Cu) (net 2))
 (segment (start 138.8 92.2) (end 138 93) (width 0.4) (layer B.Cu) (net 2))
 (segment (start 140.2 92.2) (end 139 92.2) (width 0.4) (layer B.Cu) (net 2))
 (segment (start 141.4 92.2) (end 140.2 92.2) (width 0.4) (layer F.Cu) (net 2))
 (segment (start 142.6 92.2) (end 141.4 92.2) (width 0.4) (layer F.Cu) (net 2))
 (segment (start 143.8 92.2) (end 142.6 92.2) (width 0.4) (layer B.Cu) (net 2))
 (segment (start 145 92.1) (end 143.9 92.1) (width 0.4) (layer F.Cu) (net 2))
 (segment (start 143.9 92.1) (end 143.8 92.2) (width 0.4) (layer F.Cu) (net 2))
 (segment (start 141.2 102.9) (end 141.2 102.0499) (width 0.4) (layer F.Cu) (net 2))
 (segment (start 141.2 102.0499) (end 140.8 101.6499) (width 0.4) (layer F.Cu) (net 2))
 (segment (start 140.8 101.6499) (end 140.8 98.8) (width 0.4) (layer F.Cu) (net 2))
 (segment (start 141.15 103.6012) (end 141.2 103.5512) (width 0.4) (layer F.Cu) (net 2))
 (segment (start 141.2 103.5512) (end 141.2 102.9) (width 0.4) (layer F.Cu) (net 2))
 (segment (start 141.15 105.251) (end 142.4505 105.251) (width 0.4) (layer F.Cu) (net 2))
 (segment (start 144.8 106.175) (end 143.3745 106.175) (width 0.4) (layer F.Cu) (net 2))
 (segment (start 143.3745 106.175) (end 142.4505 105.251) (width 0.4) (layer F.Cu) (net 2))
 (segment (start 141.55 96.9) (end 141.3 96.65) (width 0.4) (layer F.Cu) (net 2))
 (segment (start 141.3 96.65) (end 141.3 96.225) (width 0.4) (layer F.Cu) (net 2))
 (segment (start 141.3 97.575) (end 141.55 97.325) (width 0.4) (layer F.Cu) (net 2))
 (segment (start 141.55 97.325) (end 141.55 96.9) (width 0.4) (layer F.Cu) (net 2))
 (segment (start 138.8999 95.4) (end 138.8999 95.55) (width 0.4) (layer F.Cu) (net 2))
 (segment (start 141.3 94.875) (end 139.4249 94.875) (width 0.4) (layer F.Cu) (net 2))
 (segment (start 139.4249 94.875) (end 138.8999 95.4) (width 0.4) (layer F.Cu) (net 2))
 (segment (start 138.8999 95.4) (end 138 95.4) (width 0.4) (layer F.Cu) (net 2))
 (segment (start 141.55 95.55) (end 138.8999 95.55) (width 0.4) (layer F.Cu) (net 2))
 (segment (start 141.55 94.2) (end 141.3 94.45) (width 0.4) (layer F.Cu) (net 2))
 (segment (start 141.3 94.45) (end 141.3 94.875) (width 0.4) (layer F.Cu) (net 2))
 (segment (start 141.3 96.225) (end 141.55 95.975) (width 0.4) (layer F.Cu) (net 2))
 (segment (start 141.55 95.975) (end 141.55 95.55) (width 0.4) (layer F.Cu) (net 2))
 (segment (start 141.55 94.2) (end 141.3 93.95) (width 0.4) (layer F.Cu) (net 2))
 (segment (start 141.3 93.95) (end 141.3 93.525) (width 0.4) (layer F.Cu) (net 2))
 (segment (start 141.15 105.251) (end 141.15 103.6012) (width 0.4) (layer F.Cu) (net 2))
 (segment (start 132.4 95.4) (end 138 95.4) (width 0.4) (layer F.Cu) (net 2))
 (segment (start 153.45 108.9) (end 153.45 107.65) (width 0.4) (layer F.Cu) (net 10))
 (segment (start 153.45 107.65) (end 153.5 107.6) (width 0.4) (layer F.Cu) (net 10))
 (segment (start 146.4 95.32) (end 146.4 95.2) (width 0.4) (layer F.Cu) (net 1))
 (segment (start 146.0001 96.185) (end 146.4 95.7851) (width 0.4) (layer F.Cu) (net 1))
 (segment (start 146.4 95.7851) (end 146.4 95.32) (width 0.4) (layer F.Cu) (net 1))
 (segment (start 146.4 95.32) (end 146.6749 95.32) (width 0.4) (layer F.Cu) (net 1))
 (segment (start 147.675 95.32) (end 146.6749 95.32) (width 0.4) (layer F.Cu) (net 1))
 (segment (start 146.0001 96.185) (end 146.2151 96.4) (width 0.4) (layer F.Cu) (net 1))
 (segment (start 146.2151 96.4) (end 146.4 96.4) (width 0.4) (layer F.Cu) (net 1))
 (segment (start 145 94.915) (end 145 96.185) (width 0.4) (layer F.Cu) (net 1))
 (segment (start 147.675 96.59) (end 146.6749 96.59) (width 0.4) (layer F.Cu) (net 1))
 (segment (start 146.4 96.4) (end 146.4849 96.4) (width 0.4) (layer F.Cu) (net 1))
 (segment (start 146.4849 96.4) (end 146.6749 96.59) (width 0.4) (layer F.Cu) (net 1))
 (segment (start 147.675 97.86) (end 146.6749 97.86) (width 0.4) (layer F.Cu) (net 1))
 (segment (start 146.4 97.6) (end 146.4149 97.6) (width 0.4) (layer F.Cu) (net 1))
 (segment (start 146.4149 97.6) (end 146.6749 97.86) (width 0.4) (layer F.Cu) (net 1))
 (segment (start 146.0001 97.455) (end 146.1451 97.6) (width 0.4) (layer F.Cu) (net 1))
 (segment (start 146.1451 97.6) (end 146.4 97.6) (width 0.4) (layer F.Cu) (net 1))
 (segment (start 145 96.185) (end 146.0001 96.185) (width 0.4) (layer F.Cu) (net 1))
 (segment (start 145 97.455) (end 146.0001 97.455) (width 0.4) (layer F.Cu) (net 1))
 (segment (start 145.47 102.35) (end 144.7749 102.35) (width 0.4) (layer F.Cu) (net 1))
 (segment (start 144.8 104.875) (end 143.6749 104.875) (width 0.4) (layer F.Cu) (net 1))
 (segment (start 143.6749 104.875) (end 143.6749 103.45) (width 0.4) (layer F.Cu) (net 1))
 (segment (start 143.6749 103.45) (end 144.7749 102.35) (width 0.4) (layer F.Cu) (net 1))
 (segment (start 145.47 102.35) (end 145.47 101.7249) (width 0.4) (layer F.Cu) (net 1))
 (segment (start 145.4 99.8) (end 145.4 101.6549) (width 0.4) (layer F.Cu) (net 1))
 (segment (start 145.4 101.6549) (end 145.47 101.7249) (width 0.4) (layer F.Cu) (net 1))
 (segment (start 146.4 97.6) (end 145.4 98.6) (width 0.4) (layer B.Cu) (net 1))
 (segment (start 145.4 98.6) (end 145.4 99.8) (width 0.4) (layer B.Cu) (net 1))
 (segment (start 146.4 96.4) (end 146.4 97.6) (width 0.4) (layer B.Cu) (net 1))
 (segment (start 146.7 93.7) (end 145.055 93.7) (width 0.4) (layer F.Cu) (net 9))
 (segment (start 145.055 93.7) (end 145 93.645) (width 0.4) (layer F.Cu) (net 9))
 (segment (start 139.25 103.8) (end 139.25 103.35) (width 0.4) (layer F.Cu) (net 7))
 (segment (start 139.25 103.35) (end 139.7 102.9) (width 0.4) (layer F.Cu) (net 7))
 (segment (start 149.2 106.175) (end 147.475 106.175) (width 0.4) (layer F.Cu) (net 7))
 (segment (start 147.475 106.175) (end 146.4 107.25) (width 0.4) (layer F.Cu) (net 7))
 (segment (start 146.4 107.25) (end 139.8 107.25) (width 0.4) (layer F.Cu) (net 7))
 (segment (start 139.8 107.25) (end 139.25 106.7) (width 0.4) (layer F.Cu) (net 7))
 (segment (start 139.25 106.7) (end 139.25 103.8) (width 0.4) (layer F.Cu) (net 7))
 (segment (start 137.33 103.85) (end 139.2 103.85) (width 0.4) (layer F.Cu) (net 7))
 (segment (start 139.2 103.85) (end 139.25 103.8) (width 0.4) (layer F.Cu) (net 7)))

